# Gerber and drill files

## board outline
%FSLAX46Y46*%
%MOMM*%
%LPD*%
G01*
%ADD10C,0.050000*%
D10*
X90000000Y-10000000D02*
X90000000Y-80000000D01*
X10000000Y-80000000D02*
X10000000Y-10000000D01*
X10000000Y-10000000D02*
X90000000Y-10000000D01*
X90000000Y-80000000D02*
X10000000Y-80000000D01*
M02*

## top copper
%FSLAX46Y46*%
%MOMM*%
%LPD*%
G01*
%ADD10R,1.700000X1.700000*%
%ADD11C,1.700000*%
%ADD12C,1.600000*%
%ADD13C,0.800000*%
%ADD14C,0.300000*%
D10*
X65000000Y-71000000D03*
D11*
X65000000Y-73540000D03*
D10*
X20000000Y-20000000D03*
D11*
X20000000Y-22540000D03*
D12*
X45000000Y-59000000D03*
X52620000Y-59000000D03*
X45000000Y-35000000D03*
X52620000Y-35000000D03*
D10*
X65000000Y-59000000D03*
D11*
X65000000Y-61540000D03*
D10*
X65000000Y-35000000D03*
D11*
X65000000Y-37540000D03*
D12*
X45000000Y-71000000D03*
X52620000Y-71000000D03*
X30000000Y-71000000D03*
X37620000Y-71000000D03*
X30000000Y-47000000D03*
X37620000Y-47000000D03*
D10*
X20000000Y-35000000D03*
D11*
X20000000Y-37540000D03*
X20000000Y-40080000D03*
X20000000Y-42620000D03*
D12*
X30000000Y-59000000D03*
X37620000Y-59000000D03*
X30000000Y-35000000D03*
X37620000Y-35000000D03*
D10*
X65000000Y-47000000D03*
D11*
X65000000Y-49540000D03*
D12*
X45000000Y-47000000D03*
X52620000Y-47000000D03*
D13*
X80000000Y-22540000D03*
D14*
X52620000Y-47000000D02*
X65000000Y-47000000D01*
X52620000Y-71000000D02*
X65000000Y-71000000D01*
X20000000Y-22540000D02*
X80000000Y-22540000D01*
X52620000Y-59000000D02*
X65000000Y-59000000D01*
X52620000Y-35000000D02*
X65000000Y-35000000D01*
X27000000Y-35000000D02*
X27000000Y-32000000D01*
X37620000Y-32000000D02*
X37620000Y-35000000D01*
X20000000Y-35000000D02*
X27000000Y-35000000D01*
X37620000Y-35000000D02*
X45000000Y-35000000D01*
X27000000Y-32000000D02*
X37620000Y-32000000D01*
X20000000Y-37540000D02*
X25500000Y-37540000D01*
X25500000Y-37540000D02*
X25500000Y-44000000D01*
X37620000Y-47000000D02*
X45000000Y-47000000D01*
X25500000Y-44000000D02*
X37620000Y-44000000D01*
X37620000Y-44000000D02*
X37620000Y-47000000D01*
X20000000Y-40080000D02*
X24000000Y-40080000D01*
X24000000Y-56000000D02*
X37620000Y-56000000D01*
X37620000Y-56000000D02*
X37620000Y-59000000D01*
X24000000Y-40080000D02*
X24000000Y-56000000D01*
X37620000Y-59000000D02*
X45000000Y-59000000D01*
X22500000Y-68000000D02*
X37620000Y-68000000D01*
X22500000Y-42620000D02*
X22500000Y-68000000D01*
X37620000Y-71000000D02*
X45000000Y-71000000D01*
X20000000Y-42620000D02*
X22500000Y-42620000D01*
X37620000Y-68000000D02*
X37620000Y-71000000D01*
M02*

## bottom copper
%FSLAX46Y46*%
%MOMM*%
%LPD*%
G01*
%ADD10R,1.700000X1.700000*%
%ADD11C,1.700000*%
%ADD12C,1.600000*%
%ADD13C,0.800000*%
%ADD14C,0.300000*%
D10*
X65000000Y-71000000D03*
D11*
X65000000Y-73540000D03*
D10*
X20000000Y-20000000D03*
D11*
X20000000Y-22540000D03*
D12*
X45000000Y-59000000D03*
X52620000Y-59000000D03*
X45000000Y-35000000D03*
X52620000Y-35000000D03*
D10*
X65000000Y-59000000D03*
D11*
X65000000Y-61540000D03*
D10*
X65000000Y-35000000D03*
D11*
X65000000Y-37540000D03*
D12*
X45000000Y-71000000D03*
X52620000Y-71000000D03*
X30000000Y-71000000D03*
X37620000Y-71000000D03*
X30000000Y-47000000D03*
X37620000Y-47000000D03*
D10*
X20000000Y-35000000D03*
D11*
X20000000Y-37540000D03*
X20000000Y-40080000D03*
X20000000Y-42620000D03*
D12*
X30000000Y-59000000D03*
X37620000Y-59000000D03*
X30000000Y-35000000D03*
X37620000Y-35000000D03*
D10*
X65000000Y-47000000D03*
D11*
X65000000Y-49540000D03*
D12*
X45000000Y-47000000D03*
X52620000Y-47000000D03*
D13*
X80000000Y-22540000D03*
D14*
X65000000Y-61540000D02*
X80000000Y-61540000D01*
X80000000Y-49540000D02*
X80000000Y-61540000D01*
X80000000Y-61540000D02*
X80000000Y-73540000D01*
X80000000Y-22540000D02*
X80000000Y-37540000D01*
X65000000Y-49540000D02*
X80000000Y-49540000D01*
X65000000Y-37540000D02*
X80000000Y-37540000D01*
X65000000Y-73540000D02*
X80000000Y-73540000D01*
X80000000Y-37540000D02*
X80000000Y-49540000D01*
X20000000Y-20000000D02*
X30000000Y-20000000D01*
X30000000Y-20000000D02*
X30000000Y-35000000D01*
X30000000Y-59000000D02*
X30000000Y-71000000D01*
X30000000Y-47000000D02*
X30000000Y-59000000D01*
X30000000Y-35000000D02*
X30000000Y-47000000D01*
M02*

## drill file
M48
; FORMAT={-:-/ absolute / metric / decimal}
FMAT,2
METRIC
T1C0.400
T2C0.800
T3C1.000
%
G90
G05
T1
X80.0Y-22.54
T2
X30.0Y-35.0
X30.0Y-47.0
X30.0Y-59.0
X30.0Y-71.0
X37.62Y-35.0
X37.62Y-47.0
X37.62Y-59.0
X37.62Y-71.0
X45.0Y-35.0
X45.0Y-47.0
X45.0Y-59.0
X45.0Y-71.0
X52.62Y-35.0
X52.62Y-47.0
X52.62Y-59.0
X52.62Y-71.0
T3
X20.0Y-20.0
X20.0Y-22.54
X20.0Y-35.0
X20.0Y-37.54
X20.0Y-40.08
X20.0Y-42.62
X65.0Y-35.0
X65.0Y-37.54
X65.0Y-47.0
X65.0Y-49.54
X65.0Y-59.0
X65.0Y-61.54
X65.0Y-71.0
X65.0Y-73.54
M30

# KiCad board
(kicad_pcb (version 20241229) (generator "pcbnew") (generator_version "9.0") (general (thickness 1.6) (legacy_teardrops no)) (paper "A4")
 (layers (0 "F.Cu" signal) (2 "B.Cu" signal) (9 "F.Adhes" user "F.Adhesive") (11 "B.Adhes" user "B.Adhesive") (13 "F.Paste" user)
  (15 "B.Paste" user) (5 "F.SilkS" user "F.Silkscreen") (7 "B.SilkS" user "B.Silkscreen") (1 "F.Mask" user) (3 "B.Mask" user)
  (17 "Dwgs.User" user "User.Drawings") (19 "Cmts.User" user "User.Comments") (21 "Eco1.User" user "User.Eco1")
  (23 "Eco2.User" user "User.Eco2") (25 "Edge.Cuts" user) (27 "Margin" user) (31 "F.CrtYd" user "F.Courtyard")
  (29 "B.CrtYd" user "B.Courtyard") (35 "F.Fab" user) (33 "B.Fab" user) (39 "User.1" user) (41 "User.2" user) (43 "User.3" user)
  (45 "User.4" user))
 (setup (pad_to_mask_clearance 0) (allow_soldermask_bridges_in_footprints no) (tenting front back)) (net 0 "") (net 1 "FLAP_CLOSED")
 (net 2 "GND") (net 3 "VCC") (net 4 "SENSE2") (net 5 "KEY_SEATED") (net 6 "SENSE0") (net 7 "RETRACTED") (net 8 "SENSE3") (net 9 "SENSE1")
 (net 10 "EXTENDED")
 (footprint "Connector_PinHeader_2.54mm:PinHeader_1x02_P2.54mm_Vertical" (layer "F.Cu") (at 65 71)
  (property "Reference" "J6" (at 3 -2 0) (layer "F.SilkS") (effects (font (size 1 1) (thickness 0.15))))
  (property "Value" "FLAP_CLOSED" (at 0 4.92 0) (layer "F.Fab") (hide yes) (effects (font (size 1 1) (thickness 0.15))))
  (pad "1" thru_hole rect (at 0 0) (size 1.7 1.7) (drill 1) (layers "*.Cu" "*.Mask") (remove_unused_layers no) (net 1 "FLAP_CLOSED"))
  (pad "2" thru_hole circle (at 0 2.54) (size 1.7 1.7) (drill 1) (layers "*.Cu" "*.Mask") (remove_unused_layers no) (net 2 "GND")))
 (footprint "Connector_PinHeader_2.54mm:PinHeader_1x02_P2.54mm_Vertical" (layer "F.Cu") (at 20 20)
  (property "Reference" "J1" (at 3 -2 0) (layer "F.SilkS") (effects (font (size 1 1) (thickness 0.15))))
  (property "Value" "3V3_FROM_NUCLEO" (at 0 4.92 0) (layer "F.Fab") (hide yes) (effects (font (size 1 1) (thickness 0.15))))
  (pad "1" thru_hole rect (at 0 0) (size 1.7 1.7) (drill 1) (layers "*.Cu" "*.Mask") (remove_unused_layers no) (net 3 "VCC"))
  (pad "2" thru_hole circle (at 0 2.54) (size 1.7 1.7) (drill 1) (layers "*.Cu" "*.Mask") (remove_unused_layers no) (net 2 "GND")))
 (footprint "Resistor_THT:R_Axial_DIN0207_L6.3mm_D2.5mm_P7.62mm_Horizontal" (layer "F.Cu") (at 45 59)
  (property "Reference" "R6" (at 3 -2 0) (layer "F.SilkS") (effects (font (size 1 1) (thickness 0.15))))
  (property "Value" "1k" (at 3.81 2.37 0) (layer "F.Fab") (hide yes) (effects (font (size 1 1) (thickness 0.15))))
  (pad "1" thru_hole circle (at 0 0) (size 1.6 1.6) (drill 0.8) (layers "*.Cu" "*.Mask") (remove_unused_layers no) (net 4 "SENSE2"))
  (pad "2" thru_hole circle (at 7.62 0) (size 1.6 1.6) (drill 0.8) (layers "*.Cu" "*.Mask") (remove_unused_layers no) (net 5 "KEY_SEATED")))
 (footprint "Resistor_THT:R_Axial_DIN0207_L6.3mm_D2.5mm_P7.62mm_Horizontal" (layer "F.Cu") (at 45 35)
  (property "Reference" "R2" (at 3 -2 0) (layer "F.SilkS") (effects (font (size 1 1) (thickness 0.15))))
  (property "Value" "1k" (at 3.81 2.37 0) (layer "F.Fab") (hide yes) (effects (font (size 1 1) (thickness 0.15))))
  (pad "1" thru_hole circle (at 0 0) (size 1.6 1.6) (drill 0.8) (layers "*.Cu" "*.Mask") (remove_unused_layers no) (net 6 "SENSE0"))
  (pad "2" thru_hole circle (at 7.62 0) (size 1.6 1.6) (drill 0.8) (layers "*.Cu" "*.Mask") (remove_unused_layers no) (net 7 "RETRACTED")))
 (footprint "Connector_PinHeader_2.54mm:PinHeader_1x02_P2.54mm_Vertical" (layer "F.Cu") (at 65 59)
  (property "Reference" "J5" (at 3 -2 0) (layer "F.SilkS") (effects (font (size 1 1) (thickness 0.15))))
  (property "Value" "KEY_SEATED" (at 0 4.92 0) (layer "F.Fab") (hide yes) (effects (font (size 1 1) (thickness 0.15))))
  (pad "1" thru_hole rect (at 0 0) (size 1.7 1.7) (drill 1) (layers "*.Cu" "*.Mask") (remove_unused_layers no) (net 5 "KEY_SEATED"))
  (pad "2" thru_hole circle (at 0 2.54) (size 1.7 1.7) (drill 1) (layers "*.Cu" "*.Mask") (remove_unused_layers no) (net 2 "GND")))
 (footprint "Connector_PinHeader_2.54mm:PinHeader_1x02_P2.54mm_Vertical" (layer "F.Cu") (at 65 35)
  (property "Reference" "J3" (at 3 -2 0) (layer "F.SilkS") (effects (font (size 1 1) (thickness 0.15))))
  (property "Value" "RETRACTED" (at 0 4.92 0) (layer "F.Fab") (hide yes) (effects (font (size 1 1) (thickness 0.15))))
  (pad "1" thru_hole rect (at 0 0) (size 1.7 1.7) (drill 1) (layers "*.Cu" "*.Mask") (remove_unused_layers no) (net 7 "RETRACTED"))
  (pad "2" thru_hole circle (at 0 2.54) (size 1.7 1.7) (drill 1) (layers "*.Cu" "*.Mask") (remove_unused_layers no) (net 2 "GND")))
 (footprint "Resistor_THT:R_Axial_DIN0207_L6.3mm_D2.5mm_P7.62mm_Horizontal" (layer "F.Cu") (at 45 71)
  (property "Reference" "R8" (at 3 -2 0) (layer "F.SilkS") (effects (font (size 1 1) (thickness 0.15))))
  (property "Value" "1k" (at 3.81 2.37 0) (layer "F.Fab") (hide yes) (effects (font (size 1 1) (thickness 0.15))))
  (pad "1" thru_hole circle (at 0 0) (size 1.6 1.6) (drill 0.8) (layers "*.Cu" "*.Mask") (remove_unused_layers no) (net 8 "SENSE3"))
  (pad "2" thru_hole circle (at 7.62 0) (size 1.6 1.6) (drill 0.8) (layers "*.Cu" "*.Mask") (remove_unused_layers no) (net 1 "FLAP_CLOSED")))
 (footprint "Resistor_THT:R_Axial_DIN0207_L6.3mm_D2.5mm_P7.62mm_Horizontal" (layer "F.Cu") (at 30 71)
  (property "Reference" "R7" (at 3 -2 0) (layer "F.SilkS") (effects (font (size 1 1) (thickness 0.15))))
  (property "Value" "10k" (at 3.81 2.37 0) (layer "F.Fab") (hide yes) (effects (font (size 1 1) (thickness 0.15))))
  (pad "1" thru_hole circle (at 0 0) (size 1.6 1.6) (drill 0.8) (layers "*.Cu" "*.Mask") (remove_unused_layers no) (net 3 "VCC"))
  (pad "2" thru_hole circle (at 7.62 0) (size 1.6 1.6) (drill 0.8) (layers "*.Cu" "*.Mask") (remove_unused_layers no) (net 8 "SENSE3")))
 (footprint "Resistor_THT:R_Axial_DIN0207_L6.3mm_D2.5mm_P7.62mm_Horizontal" (layer "F.Cu") (at 30 47)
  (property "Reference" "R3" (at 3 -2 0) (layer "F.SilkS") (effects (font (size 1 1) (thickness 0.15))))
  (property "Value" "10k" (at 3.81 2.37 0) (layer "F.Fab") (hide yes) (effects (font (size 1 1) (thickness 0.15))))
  (pad "1" thru_hole circle (at 0 0) (size 1.6 1.6) (drill 0.8) (layers "*.Cu" "*.Mask") (remove_unused_layers no) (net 3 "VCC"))
  (pad "2" thru_hole circle (at 7.62 0) (size 1.6 1.6) (drill 0.8) (layers "*.Cu" "*.Mask") (remove_unused_layers no) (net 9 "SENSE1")))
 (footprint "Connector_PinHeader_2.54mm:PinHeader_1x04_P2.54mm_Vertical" (layer "F.Cu") (at 20 35)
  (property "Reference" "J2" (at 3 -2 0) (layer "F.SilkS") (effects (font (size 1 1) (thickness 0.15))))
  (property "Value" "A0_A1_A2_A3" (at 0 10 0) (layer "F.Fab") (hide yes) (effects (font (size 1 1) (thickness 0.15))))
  (pad "1" thru_hole rect (at 0 0) (size 1.7 1.7) (drill 1) (layers "*.Cu" "*.Mask") (remove_unused_layers no) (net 6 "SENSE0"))
  (pad "2" thru_hole circle (at 0 2.54) (size 1.7 1.7) (drill 1) (layers "*.Cu" "*.Mask") (remove_unused_layers no) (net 9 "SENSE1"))
  (pad "3" thru_hole circle (at 0 5.08) (size 1.7 1.7) (drill 1) (layers "*.Cu" "*.Mask") (remove_unused_layers no) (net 4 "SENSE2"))
  (pad "4" thru_hole circle (at 0 7.62) (size 1.7 1.7) (drill 1) (layers "*.Cu" "*.Mask") (remove_unused_layers no) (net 8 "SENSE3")))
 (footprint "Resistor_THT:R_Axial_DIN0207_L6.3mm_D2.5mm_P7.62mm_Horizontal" (layer "F.Cu") (at 30 59)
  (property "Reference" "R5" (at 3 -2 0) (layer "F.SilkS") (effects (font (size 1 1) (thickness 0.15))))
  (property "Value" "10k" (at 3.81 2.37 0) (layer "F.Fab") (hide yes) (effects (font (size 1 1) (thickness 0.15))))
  (pad "1" thru_hole circle (at 0 0) (size 1.6 1.6) (drill 0.8) (layers "*.Cu" "*.Mask") (remove_unused_layers no) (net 3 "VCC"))
  (pad "2" thru_hole circle (at 7.62 0) (size 1.6 1.6) (drill 0.8) (layers "*.Cu" "*.Mask") (remove_unused_layers no) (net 4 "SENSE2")))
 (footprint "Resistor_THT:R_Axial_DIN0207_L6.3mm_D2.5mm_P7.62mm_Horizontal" (layer "F.Cu") (at 30 35)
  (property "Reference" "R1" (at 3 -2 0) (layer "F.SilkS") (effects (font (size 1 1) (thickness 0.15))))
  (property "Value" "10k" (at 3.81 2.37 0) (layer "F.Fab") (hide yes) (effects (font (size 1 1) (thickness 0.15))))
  (pad "1" thru_hole circle (at 0 0) (size 1.6 1.6) (drill 0.8) (layers "*.Cu" "*.Mask") (remove_unused_layers no) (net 3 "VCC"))
  (pad "2" thru_hole circle (at 7.62 0) (size 1.6 1.6) (drill 0.8) (layers "*.Cu" "*.Mask") (remove_unused_layers no) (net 6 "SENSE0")))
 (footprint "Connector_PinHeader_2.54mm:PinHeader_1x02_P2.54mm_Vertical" (layer "F.Cu") (at 65 47)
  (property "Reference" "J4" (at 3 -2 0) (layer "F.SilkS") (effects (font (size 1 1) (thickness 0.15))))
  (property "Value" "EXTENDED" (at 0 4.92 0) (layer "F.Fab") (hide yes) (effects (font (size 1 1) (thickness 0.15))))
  (pad "1" thru_hole rect (at 0 0) (size 1.7 1.7) (drill 1) (layers "*.Cu" "*.Mask") (remove_unused_layers no) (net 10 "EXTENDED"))
  (pad "2" thru_hole circle (at 0 2.54) (size 1.7 1.7) (drill 1) (layers "*.Cu" "*.Mask") (remove_unused_layers no) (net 2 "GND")))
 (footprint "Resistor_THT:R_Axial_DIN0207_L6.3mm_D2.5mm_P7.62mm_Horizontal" (layer "F.Cu") (at 45 47)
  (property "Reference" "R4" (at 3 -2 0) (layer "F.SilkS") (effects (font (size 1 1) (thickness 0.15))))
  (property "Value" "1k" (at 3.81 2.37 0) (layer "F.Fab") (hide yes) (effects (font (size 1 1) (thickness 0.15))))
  (pad "1" thru_hole circle (at 0 0) (size 1.6 1.6) (drill 0.8) (layers "*.Cu" "*.Mask") (remove_unused_layers no) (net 9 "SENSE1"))
  (pad "2" thru_hole circle (at 7.62 0) (size 1.6 1.6) (drill 0.8) (layers "*.Cu" "*.Mask") (remove_unused_layers no) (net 10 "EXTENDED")))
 (gr_line (start 90 10) (end 90 80) (stroke (width 0.05) (type default)) (layer "Edge.Cuts"))
 (gr_line (start 10 80) (end 10 10) (stroke (width 0.05) (type default)) (layer "Edge.Cuts"))
 (gr_line (start 10 10) (end 90 10) (stroke (width 0.05) (type default)) (layer "Edge.Cuts"))
 (gr_line (start 90 80) (end 10 80) (stroke (width 0.05) (type default)) (layer "Edge.Cuts"))
 (segment (start 52.62 47) (end 65 47) (width 0.3) (layer "F.Cu") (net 10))
 (segment (start 52.62 71) (end 65 71) (width 0.3) (layer "F.Cu") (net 1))
 (segment (start 20 22.54) (end 80 22.54) (width 0.3) (layer "F.Cu") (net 2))
 (via (at 80 22.54) (size 0.8) (drill 0.4) (layers "F.Cu" "B.Cu") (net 2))
 (segment (start 65 61.54) (end 80 61.54) (width 0.3) (layer "B.Cu") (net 2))
 (segment (start 80 49.54) (end 80 61.54) (width 0.3) (layer "B.Cu") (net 2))
 (segment (start 80 61.54) (end 80 73.54) (width 0.3) (layer "B.Cu") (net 2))
 (segment (start 80 22.54) (end 80 37.54) (width 0.3) (layer "B.Cu") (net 2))
 (segment (start 65 49.54) (end 80 49.54) (width 0.3) (layer "B.Cu") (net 2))
 (segment (start 65 37.54) (end 80 37.54) (width 0.3) (layer "B.Cu") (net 2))
 (segment (start 65 73.54) (end 80 73.54) (width 0.3) (layer "B.Cu") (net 2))
 (segment (start 80 37.54) (end 80 49.54) (width 0.3) (layer "B.Cu") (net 2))
 (segment (start 52.62 59) (end 65 59) (width 0.3) (layer "F.Cu") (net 5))
 (segment (start 52.62 35) (end 65 35) (width 0.3) (layer "F.Cu") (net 7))
 (segment (start 27 35) (end 27 32) (width 0.3) (layer "F.Cu") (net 6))
 (segment (start 37.62 32) (end 37.62 35) (width 0.3) (layer "F.Cu") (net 6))
 (segment (start 20 35) (end 27 35) (width 0.3) (layer "F.Cu") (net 6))
 (segment (start 37.62 35) (end 45 35) (width 0.3) (layer "F.Cu") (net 6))
 (segment (start 27 32) (end 37.62 32) (width 0.3) (layer "F.Cu") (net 6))
 (segment (start 20 37.54) (end 25.5 37.54) (width 0.3) (layer "F.Cu") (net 9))
 (segment (start 25.5 37.54) (end 25.5 44) (width 0.3) (layer "F.Cu") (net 9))
 (segment (start 37.62 47) (end 45 47) (width 0.3) (layer "F.Cu") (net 9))
 (segment (start 25.5 44) (end 37.62 44) (width 0.3) (layer "F.Cu") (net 9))
 (segment (start 37.62 44) (end 37.62 47) (width 0.3) (layer "F.Cu") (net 9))
 (segment (start 20 40.08) (end 24 40.08) (width 0.3) (layer "F.Cu") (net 4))
 (segment (start 24 56) (end 37.62 56) (width 0.3) (layer "F.Cu") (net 4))
 (segment (start 37.62 56) (end 37.62 59) (width 0.3) (layer "F.Cu") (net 4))
 (segment (start 24 40.08) (end 24 56) (width 0.3) (layer "F.Cu") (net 4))
 (segment (start 37.62 59) (end 45 59) (width 0.3) (layer "F.Cu") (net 4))
 (segment (start 22.5 68) (end 37.62 68) (width 0.3) (layer "F.Cu") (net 8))
 (segment (start 22.5 42.62) (end 22.5 68) (width 0.3) (layer "F.Cu") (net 8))
 (segment (start 37.62 71) (end 45 71) (width 0.3) (layer "F.Cu") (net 8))
 (segment (start 20 42.62) (end 22.5 42.62) (width 0.3) (layer "F.Cu") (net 8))
 (segment (start 37.62 68) (end 37.62 71) (width 0.3) (layer "F.Cu") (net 8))
 (segment (start 20 20) (end 30 20) (width 0.3) (layer "B.Cu") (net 3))
 (segment (start 30 20) (end 30 35) (width 0.3) (layer "B.Cu") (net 3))
 (segment (start 30 59) (end 30 71) (width 0.3) (layer "B.Cu") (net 3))
 (segment (start 30 47) (end 30 59) (width 0.3) (layer "B.Cu") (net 3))
 (segment (start 30 35) (end 30 47) (width 0.3) (layer "B.Cu") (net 3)))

